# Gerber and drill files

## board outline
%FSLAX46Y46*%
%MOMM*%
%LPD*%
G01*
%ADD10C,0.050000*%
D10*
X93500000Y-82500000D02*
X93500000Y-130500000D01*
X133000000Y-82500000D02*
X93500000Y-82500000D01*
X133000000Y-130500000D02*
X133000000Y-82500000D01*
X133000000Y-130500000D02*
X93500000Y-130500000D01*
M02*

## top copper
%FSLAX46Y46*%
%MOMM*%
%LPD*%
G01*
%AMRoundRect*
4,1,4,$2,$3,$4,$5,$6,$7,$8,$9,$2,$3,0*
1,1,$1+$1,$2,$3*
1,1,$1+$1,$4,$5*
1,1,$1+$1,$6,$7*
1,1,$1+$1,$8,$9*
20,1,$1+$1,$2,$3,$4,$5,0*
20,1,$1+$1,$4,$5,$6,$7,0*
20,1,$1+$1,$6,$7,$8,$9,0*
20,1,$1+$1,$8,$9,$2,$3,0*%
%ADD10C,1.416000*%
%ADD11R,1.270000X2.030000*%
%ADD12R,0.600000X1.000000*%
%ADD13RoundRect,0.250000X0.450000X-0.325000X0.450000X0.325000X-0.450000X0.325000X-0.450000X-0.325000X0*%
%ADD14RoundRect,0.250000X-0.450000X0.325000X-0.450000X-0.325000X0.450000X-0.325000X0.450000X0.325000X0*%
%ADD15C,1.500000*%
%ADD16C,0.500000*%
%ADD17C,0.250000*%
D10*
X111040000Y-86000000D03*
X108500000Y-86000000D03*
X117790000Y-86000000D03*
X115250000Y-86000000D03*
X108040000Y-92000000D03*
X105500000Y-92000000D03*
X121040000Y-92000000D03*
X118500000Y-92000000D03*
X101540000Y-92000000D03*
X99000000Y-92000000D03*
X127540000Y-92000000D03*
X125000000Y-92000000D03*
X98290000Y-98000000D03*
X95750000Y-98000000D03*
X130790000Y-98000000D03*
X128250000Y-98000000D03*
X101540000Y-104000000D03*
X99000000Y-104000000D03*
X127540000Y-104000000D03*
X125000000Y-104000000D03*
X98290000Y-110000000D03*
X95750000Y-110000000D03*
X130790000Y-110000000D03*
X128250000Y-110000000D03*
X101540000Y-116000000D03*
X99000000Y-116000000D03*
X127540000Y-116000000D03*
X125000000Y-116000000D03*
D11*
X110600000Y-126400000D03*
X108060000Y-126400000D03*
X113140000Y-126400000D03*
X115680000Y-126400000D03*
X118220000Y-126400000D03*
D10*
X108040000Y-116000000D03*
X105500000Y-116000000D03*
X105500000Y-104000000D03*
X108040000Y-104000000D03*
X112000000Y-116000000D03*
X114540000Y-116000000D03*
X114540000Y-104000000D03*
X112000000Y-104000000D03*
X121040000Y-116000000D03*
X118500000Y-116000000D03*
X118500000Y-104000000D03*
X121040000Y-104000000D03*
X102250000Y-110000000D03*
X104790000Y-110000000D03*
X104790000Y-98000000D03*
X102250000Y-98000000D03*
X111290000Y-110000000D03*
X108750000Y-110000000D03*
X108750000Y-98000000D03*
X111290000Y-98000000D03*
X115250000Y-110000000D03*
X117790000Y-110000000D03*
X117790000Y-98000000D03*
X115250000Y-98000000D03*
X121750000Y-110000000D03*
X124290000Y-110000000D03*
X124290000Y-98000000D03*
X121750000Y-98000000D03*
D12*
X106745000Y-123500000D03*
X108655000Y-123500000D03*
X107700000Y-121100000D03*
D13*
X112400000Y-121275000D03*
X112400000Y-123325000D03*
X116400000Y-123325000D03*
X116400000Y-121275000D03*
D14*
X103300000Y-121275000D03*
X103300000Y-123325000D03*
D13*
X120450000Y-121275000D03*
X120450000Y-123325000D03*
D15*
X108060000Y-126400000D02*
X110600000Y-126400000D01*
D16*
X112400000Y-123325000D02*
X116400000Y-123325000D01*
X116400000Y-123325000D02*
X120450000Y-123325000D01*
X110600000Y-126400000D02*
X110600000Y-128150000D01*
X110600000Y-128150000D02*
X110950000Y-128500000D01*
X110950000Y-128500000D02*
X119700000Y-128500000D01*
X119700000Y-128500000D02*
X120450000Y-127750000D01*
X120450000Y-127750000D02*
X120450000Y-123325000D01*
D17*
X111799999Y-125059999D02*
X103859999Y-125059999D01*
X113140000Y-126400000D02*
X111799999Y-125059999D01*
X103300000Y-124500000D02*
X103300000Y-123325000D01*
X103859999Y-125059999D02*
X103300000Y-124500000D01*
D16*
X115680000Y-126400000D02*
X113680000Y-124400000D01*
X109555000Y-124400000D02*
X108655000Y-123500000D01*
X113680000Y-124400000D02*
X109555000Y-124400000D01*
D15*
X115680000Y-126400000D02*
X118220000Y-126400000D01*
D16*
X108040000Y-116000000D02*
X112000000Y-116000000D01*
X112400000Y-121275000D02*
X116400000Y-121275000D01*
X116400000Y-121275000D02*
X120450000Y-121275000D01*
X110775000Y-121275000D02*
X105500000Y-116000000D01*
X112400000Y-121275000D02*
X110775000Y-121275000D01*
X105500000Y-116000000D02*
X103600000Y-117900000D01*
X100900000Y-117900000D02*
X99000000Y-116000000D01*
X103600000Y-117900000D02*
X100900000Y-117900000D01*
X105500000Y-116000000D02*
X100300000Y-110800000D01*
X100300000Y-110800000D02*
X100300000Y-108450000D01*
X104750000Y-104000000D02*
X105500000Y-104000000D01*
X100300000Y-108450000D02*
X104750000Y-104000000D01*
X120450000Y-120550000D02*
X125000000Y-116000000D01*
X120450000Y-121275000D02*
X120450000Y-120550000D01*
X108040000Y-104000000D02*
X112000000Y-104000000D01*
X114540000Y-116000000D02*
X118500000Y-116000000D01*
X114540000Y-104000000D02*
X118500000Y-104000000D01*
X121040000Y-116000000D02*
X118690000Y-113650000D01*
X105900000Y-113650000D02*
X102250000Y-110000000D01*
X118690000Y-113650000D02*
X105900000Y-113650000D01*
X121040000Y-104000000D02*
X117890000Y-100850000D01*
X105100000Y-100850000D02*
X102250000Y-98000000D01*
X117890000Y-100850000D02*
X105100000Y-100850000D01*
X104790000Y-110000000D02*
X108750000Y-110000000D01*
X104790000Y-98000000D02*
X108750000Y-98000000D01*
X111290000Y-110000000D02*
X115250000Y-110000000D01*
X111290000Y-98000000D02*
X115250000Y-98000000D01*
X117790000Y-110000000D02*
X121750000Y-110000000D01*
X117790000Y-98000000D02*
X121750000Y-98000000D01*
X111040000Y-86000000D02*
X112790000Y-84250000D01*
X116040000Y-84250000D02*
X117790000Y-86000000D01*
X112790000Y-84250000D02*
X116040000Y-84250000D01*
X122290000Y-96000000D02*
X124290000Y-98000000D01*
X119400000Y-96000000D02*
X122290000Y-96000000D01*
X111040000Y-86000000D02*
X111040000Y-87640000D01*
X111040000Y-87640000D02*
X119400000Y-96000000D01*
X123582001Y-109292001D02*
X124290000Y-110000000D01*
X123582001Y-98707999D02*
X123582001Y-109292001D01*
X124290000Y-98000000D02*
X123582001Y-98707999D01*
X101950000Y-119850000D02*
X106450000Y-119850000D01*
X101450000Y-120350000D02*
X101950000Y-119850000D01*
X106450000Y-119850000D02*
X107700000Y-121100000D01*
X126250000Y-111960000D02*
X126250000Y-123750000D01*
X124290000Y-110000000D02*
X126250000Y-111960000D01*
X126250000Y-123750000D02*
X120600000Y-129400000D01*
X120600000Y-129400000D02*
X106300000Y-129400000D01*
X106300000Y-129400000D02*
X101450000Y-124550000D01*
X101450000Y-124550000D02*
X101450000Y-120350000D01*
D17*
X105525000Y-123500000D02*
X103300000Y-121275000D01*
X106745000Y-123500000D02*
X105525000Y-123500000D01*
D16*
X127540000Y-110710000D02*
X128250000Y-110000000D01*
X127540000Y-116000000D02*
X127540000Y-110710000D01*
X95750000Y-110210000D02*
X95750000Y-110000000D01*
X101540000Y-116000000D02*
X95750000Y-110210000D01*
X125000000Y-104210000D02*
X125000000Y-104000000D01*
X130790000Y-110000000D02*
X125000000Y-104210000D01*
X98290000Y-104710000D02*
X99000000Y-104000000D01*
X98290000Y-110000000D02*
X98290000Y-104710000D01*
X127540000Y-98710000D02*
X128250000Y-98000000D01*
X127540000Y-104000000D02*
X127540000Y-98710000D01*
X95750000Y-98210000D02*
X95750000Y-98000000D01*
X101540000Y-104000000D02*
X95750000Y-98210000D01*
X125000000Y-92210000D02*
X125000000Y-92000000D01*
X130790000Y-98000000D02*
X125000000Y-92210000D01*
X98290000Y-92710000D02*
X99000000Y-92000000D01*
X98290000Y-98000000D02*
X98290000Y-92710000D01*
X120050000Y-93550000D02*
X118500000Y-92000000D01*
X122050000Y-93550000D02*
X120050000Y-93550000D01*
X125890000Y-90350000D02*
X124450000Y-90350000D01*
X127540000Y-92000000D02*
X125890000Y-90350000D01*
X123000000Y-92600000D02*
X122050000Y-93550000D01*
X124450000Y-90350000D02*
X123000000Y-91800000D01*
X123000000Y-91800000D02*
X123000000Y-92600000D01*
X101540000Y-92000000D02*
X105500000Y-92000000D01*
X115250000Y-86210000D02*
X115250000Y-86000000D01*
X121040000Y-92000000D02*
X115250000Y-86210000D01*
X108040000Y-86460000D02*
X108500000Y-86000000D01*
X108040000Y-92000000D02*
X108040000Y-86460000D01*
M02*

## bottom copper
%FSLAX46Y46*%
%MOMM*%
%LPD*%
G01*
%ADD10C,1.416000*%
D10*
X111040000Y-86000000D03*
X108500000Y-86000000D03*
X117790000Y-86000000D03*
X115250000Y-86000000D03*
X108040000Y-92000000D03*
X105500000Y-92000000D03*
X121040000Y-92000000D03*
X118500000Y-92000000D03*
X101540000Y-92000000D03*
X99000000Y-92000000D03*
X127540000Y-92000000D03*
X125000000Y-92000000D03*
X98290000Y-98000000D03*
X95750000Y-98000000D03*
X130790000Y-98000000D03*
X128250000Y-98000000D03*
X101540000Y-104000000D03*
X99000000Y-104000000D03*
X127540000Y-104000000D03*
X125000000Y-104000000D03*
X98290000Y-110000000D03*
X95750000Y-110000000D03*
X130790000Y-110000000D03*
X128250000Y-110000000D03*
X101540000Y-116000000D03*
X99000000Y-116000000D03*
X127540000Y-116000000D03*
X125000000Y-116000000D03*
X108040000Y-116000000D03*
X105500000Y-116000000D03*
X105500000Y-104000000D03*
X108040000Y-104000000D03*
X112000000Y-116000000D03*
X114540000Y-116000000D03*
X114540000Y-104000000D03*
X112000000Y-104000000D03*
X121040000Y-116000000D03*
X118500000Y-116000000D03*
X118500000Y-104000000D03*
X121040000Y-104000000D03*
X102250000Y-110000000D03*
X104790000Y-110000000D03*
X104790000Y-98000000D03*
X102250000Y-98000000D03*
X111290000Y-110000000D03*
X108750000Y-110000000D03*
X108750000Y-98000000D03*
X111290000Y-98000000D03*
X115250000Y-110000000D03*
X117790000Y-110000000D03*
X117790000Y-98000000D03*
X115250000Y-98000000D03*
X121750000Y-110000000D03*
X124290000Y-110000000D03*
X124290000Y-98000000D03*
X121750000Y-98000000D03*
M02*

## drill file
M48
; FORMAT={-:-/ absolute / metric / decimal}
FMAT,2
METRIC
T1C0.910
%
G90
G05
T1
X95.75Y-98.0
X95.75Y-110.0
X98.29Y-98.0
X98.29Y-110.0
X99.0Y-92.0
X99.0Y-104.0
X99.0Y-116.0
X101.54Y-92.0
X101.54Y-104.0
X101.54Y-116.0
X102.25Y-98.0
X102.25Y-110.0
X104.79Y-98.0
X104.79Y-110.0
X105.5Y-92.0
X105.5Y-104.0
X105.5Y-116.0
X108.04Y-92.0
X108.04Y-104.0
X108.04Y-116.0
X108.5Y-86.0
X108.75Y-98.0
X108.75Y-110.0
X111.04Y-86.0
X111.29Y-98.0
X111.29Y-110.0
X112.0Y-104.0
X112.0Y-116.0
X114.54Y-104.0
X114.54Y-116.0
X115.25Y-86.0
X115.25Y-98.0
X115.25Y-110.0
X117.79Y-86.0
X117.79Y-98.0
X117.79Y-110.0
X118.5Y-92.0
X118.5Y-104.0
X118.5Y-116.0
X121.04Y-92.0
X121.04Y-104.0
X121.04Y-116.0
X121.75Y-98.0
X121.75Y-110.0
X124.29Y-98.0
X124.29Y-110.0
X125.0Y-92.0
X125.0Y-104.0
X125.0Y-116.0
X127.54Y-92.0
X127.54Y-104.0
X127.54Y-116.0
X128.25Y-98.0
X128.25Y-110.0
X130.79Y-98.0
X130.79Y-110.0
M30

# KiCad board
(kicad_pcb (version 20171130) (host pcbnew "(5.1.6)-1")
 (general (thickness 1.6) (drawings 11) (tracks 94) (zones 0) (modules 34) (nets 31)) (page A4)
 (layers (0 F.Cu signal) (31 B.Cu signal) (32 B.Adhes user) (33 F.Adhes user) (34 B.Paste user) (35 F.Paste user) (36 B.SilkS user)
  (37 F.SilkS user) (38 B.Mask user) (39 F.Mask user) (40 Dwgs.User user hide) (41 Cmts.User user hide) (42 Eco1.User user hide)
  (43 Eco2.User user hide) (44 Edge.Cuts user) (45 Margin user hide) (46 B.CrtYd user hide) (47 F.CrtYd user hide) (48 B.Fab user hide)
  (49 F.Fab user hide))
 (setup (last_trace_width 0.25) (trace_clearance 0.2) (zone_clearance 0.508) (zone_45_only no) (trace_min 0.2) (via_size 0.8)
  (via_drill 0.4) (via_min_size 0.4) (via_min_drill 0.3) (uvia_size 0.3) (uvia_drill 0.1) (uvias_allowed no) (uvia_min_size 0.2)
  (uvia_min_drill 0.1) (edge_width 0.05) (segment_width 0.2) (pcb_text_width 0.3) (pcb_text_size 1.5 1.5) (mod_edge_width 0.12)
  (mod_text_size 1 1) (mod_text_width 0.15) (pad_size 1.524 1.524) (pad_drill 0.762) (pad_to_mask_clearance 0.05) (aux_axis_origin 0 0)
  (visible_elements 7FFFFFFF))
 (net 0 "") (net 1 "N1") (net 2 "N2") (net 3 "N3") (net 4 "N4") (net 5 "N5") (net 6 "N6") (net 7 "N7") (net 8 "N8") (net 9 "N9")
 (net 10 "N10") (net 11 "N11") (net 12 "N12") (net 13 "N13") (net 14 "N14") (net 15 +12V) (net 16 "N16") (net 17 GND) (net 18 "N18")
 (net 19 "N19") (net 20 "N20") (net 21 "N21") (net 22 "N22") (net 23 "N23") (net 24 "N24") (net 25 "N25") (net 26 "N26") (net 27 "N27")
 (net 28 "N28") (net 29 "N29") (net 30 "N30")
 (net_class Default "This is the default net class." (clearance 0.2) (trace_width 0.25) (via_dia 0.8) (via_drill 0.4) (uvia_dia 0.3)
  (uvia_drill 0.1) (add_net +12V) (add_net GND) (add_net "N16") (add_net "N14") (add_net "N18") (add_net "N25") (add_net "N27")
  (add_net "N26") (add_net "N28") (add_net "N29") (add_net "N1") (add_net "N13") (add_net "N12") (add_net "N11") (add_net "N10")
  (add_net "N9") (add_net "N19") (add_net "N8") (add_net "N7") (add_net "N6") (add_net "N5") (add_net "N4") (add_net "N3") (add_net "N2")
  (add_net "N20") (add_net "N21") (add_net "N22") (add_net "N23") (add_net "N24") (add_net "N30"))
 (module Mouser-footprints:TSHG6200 (layer F.Cu) (at 108.5 86)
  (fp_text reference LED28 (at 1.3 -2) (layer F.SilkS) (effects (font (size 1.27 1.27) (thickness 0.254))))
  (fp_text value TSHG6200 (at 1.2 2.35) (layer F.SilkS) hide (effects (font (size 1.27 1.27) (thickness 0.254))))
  (pad 2 thru_hole circle (at 2.54 0) (size 1.416 1.416) (drill 0.91) (layers *.Cu *.Mask) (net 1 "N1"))
  (pad 1 thru_hole circle (at 0 0) (size 1.416 1.416) (drill 0.91) (layers *.Cu *.Mask) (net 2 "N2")))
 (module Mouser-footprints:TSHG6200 (layer F.Cu) (at 115.25 86)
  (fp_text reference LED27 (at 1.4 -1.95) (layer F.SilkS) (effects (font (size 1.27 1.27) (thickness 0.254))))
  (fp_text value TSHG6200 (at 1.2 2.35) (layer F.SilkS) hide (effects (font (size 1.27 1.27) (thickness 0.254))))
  (pad 2 thru_hole circle (at 2.54 0) (size 1.416 1.416) (drill 0.91) (layers *.Cu *.Mask) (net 1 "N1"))
  (pad 1 thru_hole circle (at 0 0) (size 1.416 1.416) (drill 0.91) (layers *.Cu *.Mask) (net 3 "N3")))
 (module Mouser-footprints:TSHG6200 (layer F.Cu) (at 105.5 92)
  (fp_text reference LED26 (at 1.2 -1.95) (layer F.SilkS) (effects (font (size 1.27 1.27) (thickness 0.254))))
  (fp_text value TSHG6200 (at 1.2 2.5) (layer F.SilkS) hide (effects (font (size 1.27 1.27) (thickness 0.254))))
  (pad 2 thru_hole circle (at 2.54 0) (size 1.416 1.416) (drill 0.91) (layers *.Cu *.Mask) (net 2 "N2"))
  (pad 1 thru_hole circle (at 0 0) (size 1.416 1.416) (drill 0.91) (layers *.Cu *.Mask) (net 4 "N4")))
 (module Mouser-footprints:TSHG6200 (layer F.Cu) (at 118.5 92)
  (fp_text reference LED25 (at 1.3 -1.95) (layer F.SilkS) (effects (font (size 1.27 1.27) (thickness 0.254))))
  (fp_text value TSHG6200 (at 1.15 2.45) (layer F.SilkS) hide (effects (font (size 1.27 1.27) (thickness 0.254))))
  (pad 2 thru_hole circle (at 2.54 0) (size 1.416 1.416) (drill 0.91) (layers *.Cu *.Mask) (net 3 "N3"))
  (pad 1 thru_hole circle (at 0 0) (size 1.416 1.416) (drill 0.91) (layers *.Cu *.Mask) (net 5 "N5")))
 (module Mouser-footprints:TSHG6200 (layer F.Cu) (at 99 92)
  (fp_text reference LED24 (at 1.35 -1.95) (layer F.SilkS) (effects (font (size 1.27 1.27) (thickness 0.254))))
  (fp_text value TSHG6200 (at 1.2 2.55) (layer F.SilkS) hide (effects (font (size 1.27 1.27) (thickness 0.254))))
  (pad 2 thru_hole circle (at 2.54 0) (size 1.416 1.416) (drill 0.91) (layers *.Cu *.Mask) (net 4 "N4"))
  (pad 1 thru_hole circle (at 0 0) (size 1.416 1.416) (drill 0.91) (layers *.Cu *.Mask) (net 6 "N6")))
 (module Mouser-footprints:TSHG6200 (layer F.Cu) (at 125 92)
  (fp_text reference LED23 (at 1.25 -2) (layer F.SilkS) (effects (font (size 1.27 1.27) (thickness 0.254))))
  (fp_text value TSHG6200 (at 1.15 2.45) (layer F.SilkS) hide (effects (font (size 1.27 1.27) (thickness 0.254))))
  (pad 2 thru_hole circle (at 2.54 0) (size 1.416 1.416) (drill 0.91) (layers *.Cu *.Mask) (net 5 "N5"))
  (pad 1 thru_hole circle (at 0 0) (size 1.416 1.416) (drill 0.91) (layers *.Cu *.Mask) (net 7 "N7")))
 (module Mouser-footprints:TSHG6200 (layer F.Cu) (at 95.75 98)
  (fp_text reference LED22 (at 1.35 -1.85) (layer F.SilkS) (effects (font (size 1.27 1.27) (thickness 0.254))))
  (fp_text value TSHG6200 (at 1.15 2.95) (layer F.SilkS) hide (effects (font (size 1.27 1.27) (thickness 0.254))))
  (pad 2 thru_hole circle (at 2.54 0) (size 1.416 1.416) (drill 0.91) (layers *.Cu *.Mask) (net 6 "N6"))
  (pad 1 thru_hole circle (at 0 0) (size 1.416 1.416) (drill 0.91) (layers *.Cu *.Mask) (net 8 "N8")))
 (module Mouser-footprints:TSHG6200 (layer F.Cu) (at 128.25 98)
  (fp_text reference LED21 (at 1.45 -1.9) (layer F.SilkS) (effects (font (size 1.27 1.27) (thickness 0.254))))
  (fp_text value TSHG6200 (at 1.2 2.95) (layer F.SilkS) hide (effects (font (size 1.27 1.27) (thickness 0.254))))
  (pad 2 thru_hole circle (at 2.54 0) (size 1.416 1.416) (drill 0.91) (layers *.Cu *.Mask) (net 7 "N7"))
  (pad 1 thru_hole circle (at 0 0) (size 1.416 1.416) (drill 0.91) (layers *.Cu *.Mask) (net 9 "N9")))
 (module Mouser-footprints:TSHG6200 (layer F.Cu) (at 99 104)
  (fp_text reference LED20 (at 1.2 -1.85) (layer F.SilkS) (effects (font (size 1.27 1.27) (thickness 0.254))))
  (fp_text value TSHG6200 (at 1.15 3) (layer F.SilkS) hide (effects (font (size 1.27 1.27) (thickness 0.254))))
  (pad 2 thru_hole circle (at 2.54 0) (size 1.416 1.416) (drill 0.91) (layers *.Cu *.Mask) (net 8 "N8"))
  (pad 1 thru_hole circle (at 0 0) (size 1.416 1.416) (drill 0.91) (layers *.Cu *.Mask) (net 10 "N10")))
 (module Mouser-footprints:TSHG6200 (layer F.Cu) (at 125 104)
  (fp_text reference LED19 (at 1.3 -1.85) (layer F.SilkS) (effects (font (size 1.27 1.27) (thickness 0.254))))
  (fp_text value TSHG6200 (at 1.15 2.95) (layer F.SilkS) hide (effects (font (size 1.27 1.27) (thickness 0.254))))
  (pad 2 thru_hole circle (at 2.54 0) (size 1.416 1.416) (drill 0.91) (layers *.Cu *.Mask) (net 9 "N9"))
  (pad 1 thru_hole circle (at 0 0) (size 1.416 1.416) (drill 0.91) (layers *.Cu *.Mask) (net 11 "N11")))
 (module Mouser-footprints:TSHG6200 (layer F.Cu) (at 95.75 110)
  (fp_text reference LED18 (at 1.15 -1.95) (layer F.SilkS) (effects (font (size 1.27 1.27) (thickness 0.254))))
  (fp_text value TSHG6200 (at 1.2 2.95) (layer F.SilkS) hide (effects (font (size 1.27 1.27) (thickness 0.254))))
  (pad 2 thru_hole circle (at 2.54 0) (size 1.416 1.416) (drill 0.91) (layers *.Cu *.Mask) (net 10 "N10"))
  (pad 1 thru_hole circle (at 0 0) (size 1.416 1.416) (drill 0.91) (layers *.Cu *.Mask) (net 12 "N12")))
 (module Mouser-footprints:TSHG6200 (layer F.Cu) (at 128.25 110)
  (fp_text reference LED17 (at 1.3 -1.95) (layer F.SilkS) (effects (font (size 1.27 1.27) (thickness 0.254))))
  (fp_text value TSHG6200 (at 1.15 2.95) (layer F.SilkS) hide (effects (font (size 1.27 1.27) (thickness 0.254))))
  (pad 2 thru_hole circle (at 2.54 0) (size 1.416 1.416) (drill 0.91) (layers *.Cu *.Mask) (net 11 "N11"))
  (pad 1 thru_hole circle (at 0 0) (size 1.416 1.416) (drill 0.91) (layers *.Cu *.Mask) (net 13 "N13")))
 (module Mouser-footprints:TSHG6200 (layer F.Cu) (at 99 116)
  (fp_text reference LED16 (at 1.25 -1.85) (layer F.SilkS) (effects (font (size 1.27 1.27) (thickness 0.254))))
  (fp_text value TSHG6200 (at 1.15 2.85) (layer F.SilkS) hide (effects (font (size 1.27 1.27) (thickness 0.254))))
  (pad 2 thru_hole circle (at 2.54 0) (size 1.416 1.416) (drill 0.91) (layers *.Cu *.Mask) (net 12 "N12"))
  (pad 1 thru_hole circle (at 0 0) (size 1.416 1.416) (drill 0.91) (layers *.Cu *.Mask) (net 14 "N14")))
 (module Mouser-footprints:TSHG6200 (layer F.Cu) (at 125 116)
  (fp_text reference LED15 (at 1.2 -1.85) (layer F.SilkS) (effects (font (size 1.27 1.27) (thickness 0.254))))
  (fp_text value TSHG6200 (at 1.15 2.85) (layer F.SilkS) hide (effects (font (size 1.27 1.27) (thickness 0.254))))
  (pad 2 thru_hole circle (at 2.54 0) (size 1.416 1.416) (drill 0.91) (layers *.Cu *.Mask) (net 13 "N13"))
  (pad 1 thru_hole circle (at 0 0) (size 1.416 1.416) (drill 0.91) (layers *.Cu *.Mask) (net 14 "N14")))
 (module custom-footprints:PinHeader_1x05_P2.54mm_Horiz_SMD (layer F.Cu) (at 110.6 126.4)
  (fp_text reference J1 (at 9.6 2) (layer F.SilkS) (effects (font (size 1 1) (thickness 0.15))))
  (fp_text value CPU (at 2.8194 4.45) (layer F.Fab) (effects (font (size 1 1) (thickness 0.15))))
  (pad 2 smd rect (at 0 0) (size 1.27 2.03) (layers F.Cu F.Paste F.Mask) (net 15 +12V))
  (pad 1 smd rect (at -2.54 0) (size 1.27 2.03) (layers F.Cu F.Paste F.Mask) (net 15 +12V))
  (pad 3 smd rect (at 2.54 0) (size 1.27 2.03) (layers F.Cu F.Paste F.Mask) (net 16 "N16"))
  (pad 4 smd rect (at 5.08 0) (size 1.27 2.03) (layers F.Cu F.Paste F.Mask) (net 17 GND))
  (pad 5 smd rect (at 7.62 0) (size 1.27 2.03) (layers F.Cu F.Paste F.Mask) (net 17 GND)))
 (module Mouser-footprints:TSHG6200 (layer F.Cu) (at 105.5 116)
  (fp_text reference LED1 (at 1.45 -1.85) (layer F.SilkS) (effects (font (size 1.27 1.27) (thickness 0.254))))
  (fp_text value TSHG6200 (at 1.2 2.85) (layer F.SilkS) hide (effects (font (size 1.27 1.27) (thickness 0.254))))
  (pad 2 thru_hole circle (at 2.54 0) (size 1.416 1.416) (drill 0.91) (layers *.Cu *.Mask) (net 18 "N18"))
  (pad 1 thru_hole circle (at 0 0) (size 1.416 1.416) (drill 0.91) (layers *.Cu *.Mask) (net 14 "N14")))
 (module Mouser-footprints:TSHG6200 (layer F.Cu) (at 105.5 104)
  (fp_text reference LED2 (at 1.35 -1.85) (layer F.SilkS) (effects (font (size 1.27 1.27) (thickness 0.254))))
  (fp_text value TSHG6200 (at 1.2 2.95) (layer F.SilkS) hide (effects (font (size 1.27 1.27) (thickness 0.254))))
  (pad 1 thru_hole circle (at 0 0) (size 1.416 1.416) (drill 0.91) (layers *.Cu *.Mask) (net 14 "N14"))
  (pad 2 thru_hole circle (at 2.54 0) (size 1.416 1.416) (drill 0.91) (layers *.Cu *.Mask) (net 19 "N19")))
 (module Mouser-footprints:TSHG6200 (layer F.Cu) (at 112 116)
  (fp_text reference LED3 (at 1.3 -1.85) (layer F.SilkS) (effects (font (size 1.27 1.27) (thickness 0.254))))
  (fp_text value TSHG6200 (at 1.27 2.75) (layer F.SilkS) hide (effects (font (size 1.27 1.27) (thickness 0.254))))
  (pad 1 thru_hole circle (at 0 0) (size 1.416 1.416) (drill 0.91) (layers *.Cu *.Mask) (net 18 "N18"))
  (pad 2 thru_hole circle (at 2.54 0) (size 1.416 1.416) (drill 0.91) (layers *.Cu *.Mask) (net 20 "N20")))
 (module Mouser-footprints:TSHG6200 (layer F.Cu) (at 112 104)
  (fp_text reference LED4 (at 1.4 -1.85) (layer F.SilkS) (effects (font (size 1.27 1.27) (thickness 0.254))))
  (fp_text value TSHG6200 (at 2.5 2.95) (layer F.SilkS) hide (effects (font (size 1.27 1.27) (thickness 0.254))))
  (pad 2 thru_hole circle (at 2.54 0) (size 1.416 1.416) (drill 0.91) (layers *.Cu *.Mask) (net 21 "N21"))
  (pad 1 thru_hole circle (at 0 0) (size 1.416 1.416) (drill 0.91) (layers *.Cu *.Mask) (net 19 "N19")))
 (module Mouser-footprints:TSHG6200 (layer F.Cu) (at 118.5 116)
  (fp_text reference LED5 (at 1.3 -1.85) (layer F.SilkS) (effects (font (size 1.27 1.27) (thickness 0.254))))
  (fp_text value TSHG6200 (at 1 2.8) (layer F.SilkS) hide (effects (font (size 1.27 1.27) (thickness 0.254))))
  (pad 2 thru_hole circle (at 2.54 0) (size 1.416 1.416) (drill 0.91) (layers *.Cu *.Mask) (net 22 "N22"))
  (pad 1 thru_hole circle (at 0 0) (size 1.416 1.416) (drill 0.91) (layers *.Cu *.Mask) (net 20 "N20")))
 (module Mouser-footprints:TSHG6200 (layer F.Cu) (at 118.5 104)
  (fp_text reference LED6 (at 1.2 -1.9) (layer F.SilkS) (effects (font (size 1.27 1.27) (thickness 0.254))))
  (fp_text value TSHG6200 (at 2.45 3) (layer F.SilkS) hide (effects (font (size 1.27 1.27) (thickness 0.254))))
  (pad 1 thru_hole circle (at 0 0) (size 1.416 1.416) (drill 0.91) (layers *.Cu *.Mask) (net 21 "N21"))
  (pad 2 thru_hole circle (at 2.54 0) (size 1.416 1.416) (drill 0.91) (layers *.Cu *.Mask) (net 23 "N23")))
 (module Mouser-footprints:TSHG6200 (layer F.Cu) (at 102.25 110)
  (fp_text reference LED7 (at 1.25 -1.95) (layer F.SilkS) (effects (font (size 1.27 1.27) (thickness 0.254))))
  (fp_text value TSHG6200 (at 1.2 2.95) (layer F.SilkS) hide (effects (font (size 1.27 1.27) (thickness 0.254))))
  (pad 1 thru_hole circle (at 0 0) (size 1.416 1.416) (drill 0.91) (layers *.Cu *.Mask) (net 22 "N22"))
  (pad 2 thru_hole circle (at 2.54 0) (size 1.416 1.416) (drill 0.91) (layers *.Cu *.Mask) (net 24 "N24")))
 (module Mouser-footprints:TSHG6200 (layer F.Cu) (at 102.25 98)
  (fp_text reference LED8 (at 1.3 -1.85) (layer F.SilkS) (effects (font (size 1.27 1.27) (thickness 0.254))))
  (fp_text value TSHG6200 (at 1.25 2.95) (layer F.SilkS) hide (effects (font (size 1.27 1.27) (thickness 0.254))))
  (pad 2 thru_hole circle (at 2.54 0) (size 1.416 1.416) (drill 0.91) (layers *.Cu *.Mask) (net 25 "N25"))
  (pad 1 thru_hole circle (at 0 0) (size 1.416 1.416) (drill 0.91) (layers *.Cu *.Mask) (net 23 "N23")))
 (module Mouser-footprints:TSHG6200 (layer F.Cu) (at 108.75 110)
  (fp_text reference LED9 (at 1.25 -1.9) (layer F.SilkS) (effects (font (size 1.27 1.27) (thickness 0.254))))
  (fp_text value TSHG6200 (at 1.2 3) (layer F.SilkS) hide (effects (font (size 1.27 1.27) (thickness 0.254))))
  (pad 2 thru_hole circle (at 2.54 0) (size 1.416 1.416) (drill 0.91) (layers *.Cu *.Mask) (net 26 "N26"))
  (pad 1 thru_hole circle (at 0 0) (size 1.416 1.416) (drill 0.91) (layers *.Cu *.Mask) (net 24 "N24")))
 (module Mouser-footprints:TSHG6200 (layer F.Cu) (at 108.75 98)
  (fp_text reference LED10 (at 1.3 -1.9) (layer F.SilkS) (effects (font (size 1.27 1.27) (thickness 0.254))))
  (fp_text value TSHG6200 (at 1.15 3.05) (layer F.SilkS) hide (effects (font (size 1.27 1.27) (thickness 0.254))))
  (pad 1 thru_hole circle (at 0 0) (size 1.416 1.416) (drill 0.91) (layers *.Cu *.Mask) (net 25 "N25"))
  (pad 2 thru_hole circle (at 2.54 0) (size 1.416 1.416) (drill 0.91) (layers *.Cu *.Mask) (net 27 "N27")))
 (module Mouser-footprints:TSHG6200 (layer F.Cu) (at 115.25 110)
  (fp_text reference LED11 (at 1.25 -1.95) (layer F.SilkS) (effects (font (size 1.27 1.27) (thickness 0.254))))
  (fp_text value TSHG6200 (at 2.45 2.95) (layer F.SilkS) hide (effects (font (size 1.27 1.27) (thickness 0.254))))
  (pad 1 thru_hole circle (at 0 0) (size 1.416 1.416) (drill 0.91) (layers *.Cu *.Mask) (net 26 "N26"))
  (pad 2 thru_hole circle (at 2.54 0) (size 1.416 1.416) (drill 0.91) (layers *.Cu *.Mask) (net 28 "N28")))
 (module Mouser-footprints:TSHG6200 (layer F.Cu) (at 115.25 98)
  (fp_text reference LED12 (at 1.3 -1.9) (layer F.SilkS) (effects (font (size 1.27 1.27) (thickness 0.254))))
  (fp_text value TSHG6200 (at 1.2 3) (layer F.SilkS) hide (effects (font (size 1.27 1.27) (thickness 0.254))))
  (pad 2 thru_hole circle (at 2.54 0) (size 1.416 1.416) (drill 0.91) (layers *.Cu *.Mask) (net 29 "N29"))
  (pad 1 thru_hole circle (at 0 0) (size 1.416 1.416) (drill 0.91) (layers *.Cu *.Mask) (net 27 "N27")))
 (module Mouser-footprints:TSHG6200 (layer F.Cu) (at 121.75 110)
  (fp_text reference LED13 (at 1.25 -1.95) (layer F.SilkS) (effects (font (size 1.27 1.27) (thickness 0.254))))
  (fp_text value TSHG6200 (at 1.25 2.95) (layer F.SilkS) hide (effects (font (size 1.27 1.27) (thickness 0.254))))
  (pad 1 thru_hole circle (at 0 0) (size 1.416 1.416) (drill 0.91) (layers *.Cu *.Mask) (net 28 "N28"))
  (pad 2 thru_hole circle (at 2.54 0) (size 1.416 1.416) (drill 0.91) (layers *.Cu *.Mask) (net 1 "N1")))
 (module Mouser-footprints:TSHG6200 (layer F.Cu) (at 121.75 98)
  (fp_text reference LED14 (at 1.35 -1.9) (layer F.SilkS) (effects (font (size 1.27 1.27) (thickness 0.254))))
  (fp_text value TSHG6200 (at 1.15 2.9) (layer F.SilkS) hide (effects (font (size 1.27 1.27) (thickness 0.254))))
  (pad 2 thru_hole circle (at 2.54 0) (size 1.416 1.416) (drill 0.91) (layers *.Cu *.Mask) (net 1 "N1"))
  (pad 1 thru_hole circle (at 0 0) (size 1.416 1.416) (drill 0.91) (layers *.Cu *.Mask) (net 29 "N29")))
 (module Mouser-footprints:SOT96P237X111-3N (layer F.Cu) (at 107.7 122.3 90)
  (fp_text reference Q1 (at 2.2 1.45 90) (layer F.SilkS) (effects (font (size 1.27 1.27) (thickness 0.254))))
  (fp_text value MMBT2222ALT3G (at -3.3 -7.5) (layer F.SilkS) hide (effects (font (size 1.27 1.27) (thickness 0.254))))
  (pad 1 smd rect (at -1.2 -0.955 180) (size 0.6 1) (layers F.Cu F.Paste F.Mask) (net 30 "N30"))
  (pad 2 smd rect (at -1.2 0.955 180) (size 0.6 1) (layers F.Cu F.Paste F.Mask) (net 17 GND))
  (pad 3 smd rect (at 1.2 0 180) (size 0.6 1) (layers F.Cu F.Paste F.Mask) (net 1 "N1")))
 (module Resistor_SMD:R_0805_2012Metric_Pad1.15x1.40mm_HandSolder (layer F.Cu) (at 112.4 122.3 90)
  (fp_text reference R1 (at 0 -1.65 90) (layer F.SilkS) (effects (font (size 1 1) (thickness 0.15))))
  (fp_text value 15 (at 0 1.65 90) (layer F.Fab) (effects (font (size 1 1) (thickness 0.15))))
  (pad 2 smd roundrect (at 1.025 0 90) (size 1.15 1.4) (layers F.Cu F.Paste F.Mask) (roundrect_rratio 0.217391) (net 14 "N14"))
  (pad 1 smd roundrect (at -1.025 0 90) (size 1.15 1.4) (layers F.Cu F.Paste F.Mask) (roundrect_rratio 0.217391) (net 15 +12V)))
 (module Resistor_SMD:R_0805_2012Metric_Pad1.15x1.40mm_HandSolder (layer F.Cu) (at 116.4 122.3 90)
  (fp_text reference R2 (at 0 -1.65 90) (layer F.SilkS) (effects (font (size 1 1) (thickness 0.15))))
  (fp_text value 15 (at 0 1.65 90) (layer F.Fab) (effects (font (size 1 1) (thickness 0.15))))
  (pad 1 smd roundrect (at -1.025 0 90) (size 1.15 1.4) (layers F.Cu F.Paste F.Mask) (roundrect_rratio 0.217391) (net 15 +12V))
  (pad 2 smd roundrect (at 1.025 0 90) (size 1.15 1.4) (layers F.Cu F.Paste F.Mask) (roundrect_rratio 0.217391) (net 14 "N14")))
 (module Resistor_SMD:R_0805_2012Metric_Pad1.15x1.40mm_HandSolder (layer F.Cu) (at 103.3 122.3 270)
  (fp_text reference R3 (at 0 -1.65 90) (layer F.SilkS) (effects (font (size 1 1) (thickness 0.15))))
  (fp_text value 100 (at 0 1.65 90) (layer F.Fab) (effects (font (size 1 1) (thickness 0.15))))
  (pad 1 smd roundrect (at -1.025 0 270) (size 1.15 1.4) (layers F.Cu F.Paste F.Mask) (roundrect_rratio 0.217391) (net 30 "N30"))
  (pad 2 smd roundrect (at 1.025 0 270) (size 1.15 1.4) (layers F.Cu F.Paste F.Mask) (roundrect_rratio 0.217391) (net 16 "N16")))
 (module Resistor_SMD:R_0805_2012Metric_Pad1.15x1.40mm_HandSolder (layer F.Cu) (at 120.45 122.3 90)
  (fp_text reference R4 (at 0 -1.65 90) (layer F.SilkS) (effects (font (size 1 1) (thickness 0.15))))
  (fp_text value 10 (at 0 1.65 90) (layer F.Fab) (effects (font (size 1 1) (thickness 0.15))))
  (pad 2 smd roundrect (at 1.025 0 90) (size 1.15 1.4) (layers F.Cu F.Paste F.Mask) (roundrect_rratio 0.217391) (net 14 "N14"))
  (pad 1 smd roundrect (at -1.025 0 90) (size 1.15 1.4) (layers F.Cu F.Paste F.Mask) (roundrect_rratio 0.217391) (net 15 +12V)))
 (gr_line (start 93.5 82.5) (end 93.5 130.5) (layer Edge.Cuts) (width 0.05))
 (gr_line (start 133 82.5) (end 93.5 82.5) (layer Edge.Cuts) (width 0.05))
 (gr_line (start 133 130.5) (end 133 82.5) (layer Edge.Cuts) (width 0.05))
 (gr_line (start 133 130.5) (end 93.5 130.5) (layer Edge.Cuts) (width 0.05))
 (segment (start 108.06 126.4) (end 110.6 126.4) (width 1.5) (layer F.Cu) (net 15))
 (segment (start 112.4 123.325) (end 116.4 123.325) (width 0.5) (layer F.Cu) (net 15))
 (segment (start 116.4 123.325) (end 120.45 123.325) (width 0.5) (layer F.Cu) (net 15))
 (segment (start 110.6 126.4) (end 110.6 128.15) (width 0.5) (layer F.Cu) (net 15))
 (segment (start 110.6 128.15) (end 110.95 128.5) (width 0.5) (layer F.Cu) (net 15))
 (segment (start 110.95 128.5) (end 119.7 128.5) (width 0.5) (layer F.Cu) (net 15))
 (segment (start 119.7 128.5) (end 120.45 127.75) (width 0.5) (layer F.Cu) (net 15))
 (segment (start 120.45 127.75) (end 120.45 123.325) (width 0.5) (layer F.Cu) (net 15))
 (segment (start 111.799999 125.059999) (end 103.859999 125.059999) (width 0.25) (layer F.Cu) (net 16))
 (segment (start 113.14 126.4) (end 111.799999 125.059999) (width 0.25) (layer F.Cu) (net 16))
 (segment (start 103.3 124.5) (end 103.3 123.325) (width 0.25) (layer F.Cu) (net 16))
 (segment (start 103.859999 125.059999) (end 103.3 124.5) (width 0.25) (layer F.Cu) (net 16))
 (segment (start 115.68 126.4) (end 113.68 124.4) (width 0.5) (layer F.Cu) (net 17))
 (segment (start 109.555 124.4) (end 108.655 123.5) (width 0.5) (layer F.Cu) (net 17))
 (segment (start 113.68 124.4) (end 109.555 124.4) (width 0.5) (layer F.Cu) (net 17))
 (segment (start 115.68 126.4) (end 118.22 126.4) (width 1.5) (layer F.Cu) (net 17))
 (segment (start 108.04 116) (end 112 116) (width 0.5) (layer F.Cu) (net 18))
 (segment (start 112.4 121.275) (end 116.4 121.275) (width 0.5) (layer F.Cu) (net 14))
 (segment (start 116.4 121.275) (end 120.45 121.275) (width 0.5) (layer F.Cu) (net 14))
 (segment (start 110.775 121.275) (end 105.5 116) (width 0.5) (layer F.Cu) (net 14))
 (segment (start 112.4 121.275) (end 110.775 121.275) (width 0.5) (layer F.Cu) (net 14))
 (segment (start 105.5 116) (end 103.6 117.9) (width 0.5) (layer F.Cu) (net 14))
 (segment (start 100.9 117.9) (end 99 116) (width 0.5) (layer F.Cu) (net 14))
 (segment (start 103.6 117.9) (end 100.9 117.9) (width 0.5) (layer F.Cu) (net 14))
 (segment (start 105.5 116) (end 100.3 110.8) (width 0.5) (layer F.Cu) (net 14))
 (segment (start 100.3 110.8) (end 100.3 108.45) (width 0.5) (layer F.Cu) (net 14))
 (segment (start 104.75 104) (end 105.5 104) (width 0.5) (layer F.Cu) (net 14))
 (segment (start 100.3 108.45) (end 104.75 104) (width 0.5) (layer F.Cu) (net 14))
 (segment (start 120.45 120.55) (end 125 116) (width 0.5) (layer F.Cu) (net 14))
 (segment (start 120.45 121.275) (end 120.45 120.55) (width 0.5) (layer F.Cu) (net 14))
 (segment (start 108.04 104) (end 112 104) (width 0.5) (layer F.Cu) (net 19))
 (segment (start 114.54 116) (end 118.5 116) (width 0.5) (layer F.Cu) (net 20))
 (segment (start 114.54 104) (end 118.5 104) (width 0.5) (layer F.Cu) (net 21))
 (segment (start 121.04 116) (end 118.69 113.65) (width 0.5) (layer F.Cu) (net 22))
 (segment (start 105.9 113.65) (end 102.25 110) (width 0.5) (layer F.Cu) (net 22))
 (segment (start 118.69 113.65) (end 105.9 113.65) (width 0.5) (layer F.Cu) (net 22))
 (segment (start 121.04 104) (end 117.89 100.85) (width 0.5) (layer F.Cu) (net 23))
 (segment (start 105.1 100.85) (end 102.25 98) (width 0.5) (layer F.Cu) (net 23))
 (segment (start 117.89 100.85) (end 105.1 100.85) (width 0.5) (layer F.Cu) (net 23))
 (segment (start 104.79 110) (end 108.75 110) (width 0.5) (layer F.Cu) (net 24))
 (segment (start 104.79 98) (end 108.75 98) (width 0.5) (layer F.Cu) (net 25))
 (segment (start 111.29 110) (end 115.25 110) (width 0.5) (layer F.Cu) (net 26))
 (segment (start 111.29 98) (end 115.25 98) (width 0.5) (layer F.Cu) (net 27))
 (segment (start 117.79 110) (end 121.75 110) (width 0.5) (layer F.Cu) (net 28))
 (segment (start 117.79 98) (end 121.75 98) (width 0.5) (layer F.Cu) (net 29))
 (segment (start 111.04 86) (end 112.79 84.25) (width 0.5) (layer F.Cu) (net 1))
 (segment (start 116.04 84.25) (end 117.79 86) (width 0.5) (layer F.Cu) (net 1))
 (segment (start 112.79 84.25) (end 116.04 84.25) (width 0.5) (layer F.Cu) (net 1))
 (segment (start 122.29 96) (end 124.29 98) (width 0.5) (layer F.Cu) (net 1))
 (segment (start 119.4 96) (end 122.29 96) (width 0.5) (layer F.Cu) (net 1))
 (segment (start 111.04 86) (end 111.04 87.64) (width 0.5) (layer F.Cu) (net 1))
 (segment (start 111.04 87.64) (end 119.4 96) (width 0.5) (layer F.Cu) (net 1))
 (segment (start 123.582001 109.292001) (end 124.29 110) (width 0.5) (layer F.Cu) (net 1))
 (segment (start 123.582001 98.707999) (end 123.582001 109.292001) (width 0.5) (layer F.Cu) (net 1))
 (segment (start 124.29 98) (end 123.582001 98.707999) (width 0.5) (layer F.Cu) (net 1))
 (segment (start 101.95 119.85) (end 106.45 119.85) (width 0.5) (layer F.Cu) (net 1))
 (segment (start 101.45 120.35) (end 101.95 119.85) (width 0.5) (layer F.Cu) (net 1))
 (segment (start 106.45 119.85) (end 107.7 121.1) (width 0.5) (layer F.Cu) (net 1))
 (segment (start 126.25 111.96) (end 126.25 123.75) (width 0.5) (layer F.Cu) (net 1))
 (segment (start 124.29 110) (end 126.25 111.96) (width 0.5) (layer F.Cu) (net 1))
 (segment (start 126.25 123.75) (end 120.6 129.4) (width 0.5) (layer F.Cu) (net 1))
 (segment (start 120.6 129.4) (end 106.3 129.4) (width 0.5) (layer F.Cu) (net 1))
 (segment (start 106.3 129.4) (end 101.45 124.55) (width 0.5) (layer F.Cu) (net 1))
 (segment (start 101.45 124.55) (end 101.45 120.35) (width 0.5) (layer F.Cu) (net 1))
 (segment (start 105.525 123.5) (end 103.3 121.275) (width 0.25) (layer F.Cu) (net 30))
 (segment (start 106.745 123.5) (end 105.525 123.5) (width 0.25) (layer F.Cu) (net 30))
 (segment (start 127.54 110.71) (end 128.25 110) (width 0.5) (layer F.Cu) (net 13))
 (segment (start 127.54 116) (end 127.54 110.71) (width 0.5) (layer F.Cu) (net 13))
 (segment (start 95.75 110.21) (end 95.75 110) (width 0.5) (layer F.Cu) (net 12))
 (segment (start 101.54 116) (end 95.75 110.21) (width 0.5) (layer F.Cu) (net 12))
 (segment (start 125 104.21) (end 125 104) (width 0.5) (layer F.Cu) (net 11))
 (segment (start 130.79 110) (end 125 104.21) (width 0.5) (layer F.Cu) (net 11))
 (segment (start 98.29 104.71) (end 99 104) (width 0.5) (layer F.Cu) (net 10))
 (segment (start 98.29 110) (end 98.29 104.71) (width 0.5) (layer F.Cu) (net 10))
 (segment (start 127.54 98.71) (end 128.25 98) (width 0.5) (layer F.Cu) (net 9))
 (segment (start 127.54 104) (end 127.54 98.71) (width 0.5) (layer F.Cu) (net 9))
 (segment (start 95.75 98.21) (end 95.75 98) (width 0.5) (layer F.Cu) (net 8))
 (segment (start 101.54 104) (end 95.75 98.21) (width 0.5) (layer F.Cu) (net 8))
 (segment (start 125 92.21) (end 125 92) (width 0.5) (layer F.Cu) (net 7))
 (segment (start 130.79 98) (end 125 92.21) (width 0.5) (layer F.Cu) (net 7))
 (segment (start 98.29 92.71) (end 99 92) (width 0.5) (layer F.Cu) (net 6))
 (segment (start 98.29 98) (end 98.29 92.71) (width 0.5) (layer F.Cu) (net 6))
 (segment (start 120.05 93.55) (end 118.5 92) (width 0.5) (layer F.Cu) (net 5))
 (segment (start 122.05 93.55) (end 120.05 93.55) (width 0.5) (layer F.Cu) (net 5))
 (segment (start 125.89 90.35) (end 124.45 90.35) (width 0.5) (layer F.Cu) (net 5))
 (segment (start 127.54 92) (end 125.89 90.35) (width 0.5) (layer F.Cu) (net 5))
 (segment (start 123 92.6) (end 122.05 93.55) (width 0.5) (layer F.Cu) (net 5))
 (segment (start 124.45 90.35) (end 123 91.8) (width 0.5) (layer F.Cu) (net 5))
 (segment (start 123 91.8) (end 123 92.6) (width 0.5) (layer F.Cu) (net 5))
 (segment (start 101.54 92) (end 105.5 92) (width 0.5) (layer F.Cu) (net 4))
 (segment (start 115.25 86.21) (end 115.25 86) (width 0.5) (layer F.Cu) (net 3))
 (segment (start 121.04 92) (end 115.25 86.21) (width 0.5) (layer F.Cu) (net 3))
 (segment (start 108.04 86.46) (end 108.5 86) (width 0.5) (layer F.Cu) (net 2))
 (segment (start 108.04 92) (end 108.04 86.46) (width 0.5) (layer F.Cu) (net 2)))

